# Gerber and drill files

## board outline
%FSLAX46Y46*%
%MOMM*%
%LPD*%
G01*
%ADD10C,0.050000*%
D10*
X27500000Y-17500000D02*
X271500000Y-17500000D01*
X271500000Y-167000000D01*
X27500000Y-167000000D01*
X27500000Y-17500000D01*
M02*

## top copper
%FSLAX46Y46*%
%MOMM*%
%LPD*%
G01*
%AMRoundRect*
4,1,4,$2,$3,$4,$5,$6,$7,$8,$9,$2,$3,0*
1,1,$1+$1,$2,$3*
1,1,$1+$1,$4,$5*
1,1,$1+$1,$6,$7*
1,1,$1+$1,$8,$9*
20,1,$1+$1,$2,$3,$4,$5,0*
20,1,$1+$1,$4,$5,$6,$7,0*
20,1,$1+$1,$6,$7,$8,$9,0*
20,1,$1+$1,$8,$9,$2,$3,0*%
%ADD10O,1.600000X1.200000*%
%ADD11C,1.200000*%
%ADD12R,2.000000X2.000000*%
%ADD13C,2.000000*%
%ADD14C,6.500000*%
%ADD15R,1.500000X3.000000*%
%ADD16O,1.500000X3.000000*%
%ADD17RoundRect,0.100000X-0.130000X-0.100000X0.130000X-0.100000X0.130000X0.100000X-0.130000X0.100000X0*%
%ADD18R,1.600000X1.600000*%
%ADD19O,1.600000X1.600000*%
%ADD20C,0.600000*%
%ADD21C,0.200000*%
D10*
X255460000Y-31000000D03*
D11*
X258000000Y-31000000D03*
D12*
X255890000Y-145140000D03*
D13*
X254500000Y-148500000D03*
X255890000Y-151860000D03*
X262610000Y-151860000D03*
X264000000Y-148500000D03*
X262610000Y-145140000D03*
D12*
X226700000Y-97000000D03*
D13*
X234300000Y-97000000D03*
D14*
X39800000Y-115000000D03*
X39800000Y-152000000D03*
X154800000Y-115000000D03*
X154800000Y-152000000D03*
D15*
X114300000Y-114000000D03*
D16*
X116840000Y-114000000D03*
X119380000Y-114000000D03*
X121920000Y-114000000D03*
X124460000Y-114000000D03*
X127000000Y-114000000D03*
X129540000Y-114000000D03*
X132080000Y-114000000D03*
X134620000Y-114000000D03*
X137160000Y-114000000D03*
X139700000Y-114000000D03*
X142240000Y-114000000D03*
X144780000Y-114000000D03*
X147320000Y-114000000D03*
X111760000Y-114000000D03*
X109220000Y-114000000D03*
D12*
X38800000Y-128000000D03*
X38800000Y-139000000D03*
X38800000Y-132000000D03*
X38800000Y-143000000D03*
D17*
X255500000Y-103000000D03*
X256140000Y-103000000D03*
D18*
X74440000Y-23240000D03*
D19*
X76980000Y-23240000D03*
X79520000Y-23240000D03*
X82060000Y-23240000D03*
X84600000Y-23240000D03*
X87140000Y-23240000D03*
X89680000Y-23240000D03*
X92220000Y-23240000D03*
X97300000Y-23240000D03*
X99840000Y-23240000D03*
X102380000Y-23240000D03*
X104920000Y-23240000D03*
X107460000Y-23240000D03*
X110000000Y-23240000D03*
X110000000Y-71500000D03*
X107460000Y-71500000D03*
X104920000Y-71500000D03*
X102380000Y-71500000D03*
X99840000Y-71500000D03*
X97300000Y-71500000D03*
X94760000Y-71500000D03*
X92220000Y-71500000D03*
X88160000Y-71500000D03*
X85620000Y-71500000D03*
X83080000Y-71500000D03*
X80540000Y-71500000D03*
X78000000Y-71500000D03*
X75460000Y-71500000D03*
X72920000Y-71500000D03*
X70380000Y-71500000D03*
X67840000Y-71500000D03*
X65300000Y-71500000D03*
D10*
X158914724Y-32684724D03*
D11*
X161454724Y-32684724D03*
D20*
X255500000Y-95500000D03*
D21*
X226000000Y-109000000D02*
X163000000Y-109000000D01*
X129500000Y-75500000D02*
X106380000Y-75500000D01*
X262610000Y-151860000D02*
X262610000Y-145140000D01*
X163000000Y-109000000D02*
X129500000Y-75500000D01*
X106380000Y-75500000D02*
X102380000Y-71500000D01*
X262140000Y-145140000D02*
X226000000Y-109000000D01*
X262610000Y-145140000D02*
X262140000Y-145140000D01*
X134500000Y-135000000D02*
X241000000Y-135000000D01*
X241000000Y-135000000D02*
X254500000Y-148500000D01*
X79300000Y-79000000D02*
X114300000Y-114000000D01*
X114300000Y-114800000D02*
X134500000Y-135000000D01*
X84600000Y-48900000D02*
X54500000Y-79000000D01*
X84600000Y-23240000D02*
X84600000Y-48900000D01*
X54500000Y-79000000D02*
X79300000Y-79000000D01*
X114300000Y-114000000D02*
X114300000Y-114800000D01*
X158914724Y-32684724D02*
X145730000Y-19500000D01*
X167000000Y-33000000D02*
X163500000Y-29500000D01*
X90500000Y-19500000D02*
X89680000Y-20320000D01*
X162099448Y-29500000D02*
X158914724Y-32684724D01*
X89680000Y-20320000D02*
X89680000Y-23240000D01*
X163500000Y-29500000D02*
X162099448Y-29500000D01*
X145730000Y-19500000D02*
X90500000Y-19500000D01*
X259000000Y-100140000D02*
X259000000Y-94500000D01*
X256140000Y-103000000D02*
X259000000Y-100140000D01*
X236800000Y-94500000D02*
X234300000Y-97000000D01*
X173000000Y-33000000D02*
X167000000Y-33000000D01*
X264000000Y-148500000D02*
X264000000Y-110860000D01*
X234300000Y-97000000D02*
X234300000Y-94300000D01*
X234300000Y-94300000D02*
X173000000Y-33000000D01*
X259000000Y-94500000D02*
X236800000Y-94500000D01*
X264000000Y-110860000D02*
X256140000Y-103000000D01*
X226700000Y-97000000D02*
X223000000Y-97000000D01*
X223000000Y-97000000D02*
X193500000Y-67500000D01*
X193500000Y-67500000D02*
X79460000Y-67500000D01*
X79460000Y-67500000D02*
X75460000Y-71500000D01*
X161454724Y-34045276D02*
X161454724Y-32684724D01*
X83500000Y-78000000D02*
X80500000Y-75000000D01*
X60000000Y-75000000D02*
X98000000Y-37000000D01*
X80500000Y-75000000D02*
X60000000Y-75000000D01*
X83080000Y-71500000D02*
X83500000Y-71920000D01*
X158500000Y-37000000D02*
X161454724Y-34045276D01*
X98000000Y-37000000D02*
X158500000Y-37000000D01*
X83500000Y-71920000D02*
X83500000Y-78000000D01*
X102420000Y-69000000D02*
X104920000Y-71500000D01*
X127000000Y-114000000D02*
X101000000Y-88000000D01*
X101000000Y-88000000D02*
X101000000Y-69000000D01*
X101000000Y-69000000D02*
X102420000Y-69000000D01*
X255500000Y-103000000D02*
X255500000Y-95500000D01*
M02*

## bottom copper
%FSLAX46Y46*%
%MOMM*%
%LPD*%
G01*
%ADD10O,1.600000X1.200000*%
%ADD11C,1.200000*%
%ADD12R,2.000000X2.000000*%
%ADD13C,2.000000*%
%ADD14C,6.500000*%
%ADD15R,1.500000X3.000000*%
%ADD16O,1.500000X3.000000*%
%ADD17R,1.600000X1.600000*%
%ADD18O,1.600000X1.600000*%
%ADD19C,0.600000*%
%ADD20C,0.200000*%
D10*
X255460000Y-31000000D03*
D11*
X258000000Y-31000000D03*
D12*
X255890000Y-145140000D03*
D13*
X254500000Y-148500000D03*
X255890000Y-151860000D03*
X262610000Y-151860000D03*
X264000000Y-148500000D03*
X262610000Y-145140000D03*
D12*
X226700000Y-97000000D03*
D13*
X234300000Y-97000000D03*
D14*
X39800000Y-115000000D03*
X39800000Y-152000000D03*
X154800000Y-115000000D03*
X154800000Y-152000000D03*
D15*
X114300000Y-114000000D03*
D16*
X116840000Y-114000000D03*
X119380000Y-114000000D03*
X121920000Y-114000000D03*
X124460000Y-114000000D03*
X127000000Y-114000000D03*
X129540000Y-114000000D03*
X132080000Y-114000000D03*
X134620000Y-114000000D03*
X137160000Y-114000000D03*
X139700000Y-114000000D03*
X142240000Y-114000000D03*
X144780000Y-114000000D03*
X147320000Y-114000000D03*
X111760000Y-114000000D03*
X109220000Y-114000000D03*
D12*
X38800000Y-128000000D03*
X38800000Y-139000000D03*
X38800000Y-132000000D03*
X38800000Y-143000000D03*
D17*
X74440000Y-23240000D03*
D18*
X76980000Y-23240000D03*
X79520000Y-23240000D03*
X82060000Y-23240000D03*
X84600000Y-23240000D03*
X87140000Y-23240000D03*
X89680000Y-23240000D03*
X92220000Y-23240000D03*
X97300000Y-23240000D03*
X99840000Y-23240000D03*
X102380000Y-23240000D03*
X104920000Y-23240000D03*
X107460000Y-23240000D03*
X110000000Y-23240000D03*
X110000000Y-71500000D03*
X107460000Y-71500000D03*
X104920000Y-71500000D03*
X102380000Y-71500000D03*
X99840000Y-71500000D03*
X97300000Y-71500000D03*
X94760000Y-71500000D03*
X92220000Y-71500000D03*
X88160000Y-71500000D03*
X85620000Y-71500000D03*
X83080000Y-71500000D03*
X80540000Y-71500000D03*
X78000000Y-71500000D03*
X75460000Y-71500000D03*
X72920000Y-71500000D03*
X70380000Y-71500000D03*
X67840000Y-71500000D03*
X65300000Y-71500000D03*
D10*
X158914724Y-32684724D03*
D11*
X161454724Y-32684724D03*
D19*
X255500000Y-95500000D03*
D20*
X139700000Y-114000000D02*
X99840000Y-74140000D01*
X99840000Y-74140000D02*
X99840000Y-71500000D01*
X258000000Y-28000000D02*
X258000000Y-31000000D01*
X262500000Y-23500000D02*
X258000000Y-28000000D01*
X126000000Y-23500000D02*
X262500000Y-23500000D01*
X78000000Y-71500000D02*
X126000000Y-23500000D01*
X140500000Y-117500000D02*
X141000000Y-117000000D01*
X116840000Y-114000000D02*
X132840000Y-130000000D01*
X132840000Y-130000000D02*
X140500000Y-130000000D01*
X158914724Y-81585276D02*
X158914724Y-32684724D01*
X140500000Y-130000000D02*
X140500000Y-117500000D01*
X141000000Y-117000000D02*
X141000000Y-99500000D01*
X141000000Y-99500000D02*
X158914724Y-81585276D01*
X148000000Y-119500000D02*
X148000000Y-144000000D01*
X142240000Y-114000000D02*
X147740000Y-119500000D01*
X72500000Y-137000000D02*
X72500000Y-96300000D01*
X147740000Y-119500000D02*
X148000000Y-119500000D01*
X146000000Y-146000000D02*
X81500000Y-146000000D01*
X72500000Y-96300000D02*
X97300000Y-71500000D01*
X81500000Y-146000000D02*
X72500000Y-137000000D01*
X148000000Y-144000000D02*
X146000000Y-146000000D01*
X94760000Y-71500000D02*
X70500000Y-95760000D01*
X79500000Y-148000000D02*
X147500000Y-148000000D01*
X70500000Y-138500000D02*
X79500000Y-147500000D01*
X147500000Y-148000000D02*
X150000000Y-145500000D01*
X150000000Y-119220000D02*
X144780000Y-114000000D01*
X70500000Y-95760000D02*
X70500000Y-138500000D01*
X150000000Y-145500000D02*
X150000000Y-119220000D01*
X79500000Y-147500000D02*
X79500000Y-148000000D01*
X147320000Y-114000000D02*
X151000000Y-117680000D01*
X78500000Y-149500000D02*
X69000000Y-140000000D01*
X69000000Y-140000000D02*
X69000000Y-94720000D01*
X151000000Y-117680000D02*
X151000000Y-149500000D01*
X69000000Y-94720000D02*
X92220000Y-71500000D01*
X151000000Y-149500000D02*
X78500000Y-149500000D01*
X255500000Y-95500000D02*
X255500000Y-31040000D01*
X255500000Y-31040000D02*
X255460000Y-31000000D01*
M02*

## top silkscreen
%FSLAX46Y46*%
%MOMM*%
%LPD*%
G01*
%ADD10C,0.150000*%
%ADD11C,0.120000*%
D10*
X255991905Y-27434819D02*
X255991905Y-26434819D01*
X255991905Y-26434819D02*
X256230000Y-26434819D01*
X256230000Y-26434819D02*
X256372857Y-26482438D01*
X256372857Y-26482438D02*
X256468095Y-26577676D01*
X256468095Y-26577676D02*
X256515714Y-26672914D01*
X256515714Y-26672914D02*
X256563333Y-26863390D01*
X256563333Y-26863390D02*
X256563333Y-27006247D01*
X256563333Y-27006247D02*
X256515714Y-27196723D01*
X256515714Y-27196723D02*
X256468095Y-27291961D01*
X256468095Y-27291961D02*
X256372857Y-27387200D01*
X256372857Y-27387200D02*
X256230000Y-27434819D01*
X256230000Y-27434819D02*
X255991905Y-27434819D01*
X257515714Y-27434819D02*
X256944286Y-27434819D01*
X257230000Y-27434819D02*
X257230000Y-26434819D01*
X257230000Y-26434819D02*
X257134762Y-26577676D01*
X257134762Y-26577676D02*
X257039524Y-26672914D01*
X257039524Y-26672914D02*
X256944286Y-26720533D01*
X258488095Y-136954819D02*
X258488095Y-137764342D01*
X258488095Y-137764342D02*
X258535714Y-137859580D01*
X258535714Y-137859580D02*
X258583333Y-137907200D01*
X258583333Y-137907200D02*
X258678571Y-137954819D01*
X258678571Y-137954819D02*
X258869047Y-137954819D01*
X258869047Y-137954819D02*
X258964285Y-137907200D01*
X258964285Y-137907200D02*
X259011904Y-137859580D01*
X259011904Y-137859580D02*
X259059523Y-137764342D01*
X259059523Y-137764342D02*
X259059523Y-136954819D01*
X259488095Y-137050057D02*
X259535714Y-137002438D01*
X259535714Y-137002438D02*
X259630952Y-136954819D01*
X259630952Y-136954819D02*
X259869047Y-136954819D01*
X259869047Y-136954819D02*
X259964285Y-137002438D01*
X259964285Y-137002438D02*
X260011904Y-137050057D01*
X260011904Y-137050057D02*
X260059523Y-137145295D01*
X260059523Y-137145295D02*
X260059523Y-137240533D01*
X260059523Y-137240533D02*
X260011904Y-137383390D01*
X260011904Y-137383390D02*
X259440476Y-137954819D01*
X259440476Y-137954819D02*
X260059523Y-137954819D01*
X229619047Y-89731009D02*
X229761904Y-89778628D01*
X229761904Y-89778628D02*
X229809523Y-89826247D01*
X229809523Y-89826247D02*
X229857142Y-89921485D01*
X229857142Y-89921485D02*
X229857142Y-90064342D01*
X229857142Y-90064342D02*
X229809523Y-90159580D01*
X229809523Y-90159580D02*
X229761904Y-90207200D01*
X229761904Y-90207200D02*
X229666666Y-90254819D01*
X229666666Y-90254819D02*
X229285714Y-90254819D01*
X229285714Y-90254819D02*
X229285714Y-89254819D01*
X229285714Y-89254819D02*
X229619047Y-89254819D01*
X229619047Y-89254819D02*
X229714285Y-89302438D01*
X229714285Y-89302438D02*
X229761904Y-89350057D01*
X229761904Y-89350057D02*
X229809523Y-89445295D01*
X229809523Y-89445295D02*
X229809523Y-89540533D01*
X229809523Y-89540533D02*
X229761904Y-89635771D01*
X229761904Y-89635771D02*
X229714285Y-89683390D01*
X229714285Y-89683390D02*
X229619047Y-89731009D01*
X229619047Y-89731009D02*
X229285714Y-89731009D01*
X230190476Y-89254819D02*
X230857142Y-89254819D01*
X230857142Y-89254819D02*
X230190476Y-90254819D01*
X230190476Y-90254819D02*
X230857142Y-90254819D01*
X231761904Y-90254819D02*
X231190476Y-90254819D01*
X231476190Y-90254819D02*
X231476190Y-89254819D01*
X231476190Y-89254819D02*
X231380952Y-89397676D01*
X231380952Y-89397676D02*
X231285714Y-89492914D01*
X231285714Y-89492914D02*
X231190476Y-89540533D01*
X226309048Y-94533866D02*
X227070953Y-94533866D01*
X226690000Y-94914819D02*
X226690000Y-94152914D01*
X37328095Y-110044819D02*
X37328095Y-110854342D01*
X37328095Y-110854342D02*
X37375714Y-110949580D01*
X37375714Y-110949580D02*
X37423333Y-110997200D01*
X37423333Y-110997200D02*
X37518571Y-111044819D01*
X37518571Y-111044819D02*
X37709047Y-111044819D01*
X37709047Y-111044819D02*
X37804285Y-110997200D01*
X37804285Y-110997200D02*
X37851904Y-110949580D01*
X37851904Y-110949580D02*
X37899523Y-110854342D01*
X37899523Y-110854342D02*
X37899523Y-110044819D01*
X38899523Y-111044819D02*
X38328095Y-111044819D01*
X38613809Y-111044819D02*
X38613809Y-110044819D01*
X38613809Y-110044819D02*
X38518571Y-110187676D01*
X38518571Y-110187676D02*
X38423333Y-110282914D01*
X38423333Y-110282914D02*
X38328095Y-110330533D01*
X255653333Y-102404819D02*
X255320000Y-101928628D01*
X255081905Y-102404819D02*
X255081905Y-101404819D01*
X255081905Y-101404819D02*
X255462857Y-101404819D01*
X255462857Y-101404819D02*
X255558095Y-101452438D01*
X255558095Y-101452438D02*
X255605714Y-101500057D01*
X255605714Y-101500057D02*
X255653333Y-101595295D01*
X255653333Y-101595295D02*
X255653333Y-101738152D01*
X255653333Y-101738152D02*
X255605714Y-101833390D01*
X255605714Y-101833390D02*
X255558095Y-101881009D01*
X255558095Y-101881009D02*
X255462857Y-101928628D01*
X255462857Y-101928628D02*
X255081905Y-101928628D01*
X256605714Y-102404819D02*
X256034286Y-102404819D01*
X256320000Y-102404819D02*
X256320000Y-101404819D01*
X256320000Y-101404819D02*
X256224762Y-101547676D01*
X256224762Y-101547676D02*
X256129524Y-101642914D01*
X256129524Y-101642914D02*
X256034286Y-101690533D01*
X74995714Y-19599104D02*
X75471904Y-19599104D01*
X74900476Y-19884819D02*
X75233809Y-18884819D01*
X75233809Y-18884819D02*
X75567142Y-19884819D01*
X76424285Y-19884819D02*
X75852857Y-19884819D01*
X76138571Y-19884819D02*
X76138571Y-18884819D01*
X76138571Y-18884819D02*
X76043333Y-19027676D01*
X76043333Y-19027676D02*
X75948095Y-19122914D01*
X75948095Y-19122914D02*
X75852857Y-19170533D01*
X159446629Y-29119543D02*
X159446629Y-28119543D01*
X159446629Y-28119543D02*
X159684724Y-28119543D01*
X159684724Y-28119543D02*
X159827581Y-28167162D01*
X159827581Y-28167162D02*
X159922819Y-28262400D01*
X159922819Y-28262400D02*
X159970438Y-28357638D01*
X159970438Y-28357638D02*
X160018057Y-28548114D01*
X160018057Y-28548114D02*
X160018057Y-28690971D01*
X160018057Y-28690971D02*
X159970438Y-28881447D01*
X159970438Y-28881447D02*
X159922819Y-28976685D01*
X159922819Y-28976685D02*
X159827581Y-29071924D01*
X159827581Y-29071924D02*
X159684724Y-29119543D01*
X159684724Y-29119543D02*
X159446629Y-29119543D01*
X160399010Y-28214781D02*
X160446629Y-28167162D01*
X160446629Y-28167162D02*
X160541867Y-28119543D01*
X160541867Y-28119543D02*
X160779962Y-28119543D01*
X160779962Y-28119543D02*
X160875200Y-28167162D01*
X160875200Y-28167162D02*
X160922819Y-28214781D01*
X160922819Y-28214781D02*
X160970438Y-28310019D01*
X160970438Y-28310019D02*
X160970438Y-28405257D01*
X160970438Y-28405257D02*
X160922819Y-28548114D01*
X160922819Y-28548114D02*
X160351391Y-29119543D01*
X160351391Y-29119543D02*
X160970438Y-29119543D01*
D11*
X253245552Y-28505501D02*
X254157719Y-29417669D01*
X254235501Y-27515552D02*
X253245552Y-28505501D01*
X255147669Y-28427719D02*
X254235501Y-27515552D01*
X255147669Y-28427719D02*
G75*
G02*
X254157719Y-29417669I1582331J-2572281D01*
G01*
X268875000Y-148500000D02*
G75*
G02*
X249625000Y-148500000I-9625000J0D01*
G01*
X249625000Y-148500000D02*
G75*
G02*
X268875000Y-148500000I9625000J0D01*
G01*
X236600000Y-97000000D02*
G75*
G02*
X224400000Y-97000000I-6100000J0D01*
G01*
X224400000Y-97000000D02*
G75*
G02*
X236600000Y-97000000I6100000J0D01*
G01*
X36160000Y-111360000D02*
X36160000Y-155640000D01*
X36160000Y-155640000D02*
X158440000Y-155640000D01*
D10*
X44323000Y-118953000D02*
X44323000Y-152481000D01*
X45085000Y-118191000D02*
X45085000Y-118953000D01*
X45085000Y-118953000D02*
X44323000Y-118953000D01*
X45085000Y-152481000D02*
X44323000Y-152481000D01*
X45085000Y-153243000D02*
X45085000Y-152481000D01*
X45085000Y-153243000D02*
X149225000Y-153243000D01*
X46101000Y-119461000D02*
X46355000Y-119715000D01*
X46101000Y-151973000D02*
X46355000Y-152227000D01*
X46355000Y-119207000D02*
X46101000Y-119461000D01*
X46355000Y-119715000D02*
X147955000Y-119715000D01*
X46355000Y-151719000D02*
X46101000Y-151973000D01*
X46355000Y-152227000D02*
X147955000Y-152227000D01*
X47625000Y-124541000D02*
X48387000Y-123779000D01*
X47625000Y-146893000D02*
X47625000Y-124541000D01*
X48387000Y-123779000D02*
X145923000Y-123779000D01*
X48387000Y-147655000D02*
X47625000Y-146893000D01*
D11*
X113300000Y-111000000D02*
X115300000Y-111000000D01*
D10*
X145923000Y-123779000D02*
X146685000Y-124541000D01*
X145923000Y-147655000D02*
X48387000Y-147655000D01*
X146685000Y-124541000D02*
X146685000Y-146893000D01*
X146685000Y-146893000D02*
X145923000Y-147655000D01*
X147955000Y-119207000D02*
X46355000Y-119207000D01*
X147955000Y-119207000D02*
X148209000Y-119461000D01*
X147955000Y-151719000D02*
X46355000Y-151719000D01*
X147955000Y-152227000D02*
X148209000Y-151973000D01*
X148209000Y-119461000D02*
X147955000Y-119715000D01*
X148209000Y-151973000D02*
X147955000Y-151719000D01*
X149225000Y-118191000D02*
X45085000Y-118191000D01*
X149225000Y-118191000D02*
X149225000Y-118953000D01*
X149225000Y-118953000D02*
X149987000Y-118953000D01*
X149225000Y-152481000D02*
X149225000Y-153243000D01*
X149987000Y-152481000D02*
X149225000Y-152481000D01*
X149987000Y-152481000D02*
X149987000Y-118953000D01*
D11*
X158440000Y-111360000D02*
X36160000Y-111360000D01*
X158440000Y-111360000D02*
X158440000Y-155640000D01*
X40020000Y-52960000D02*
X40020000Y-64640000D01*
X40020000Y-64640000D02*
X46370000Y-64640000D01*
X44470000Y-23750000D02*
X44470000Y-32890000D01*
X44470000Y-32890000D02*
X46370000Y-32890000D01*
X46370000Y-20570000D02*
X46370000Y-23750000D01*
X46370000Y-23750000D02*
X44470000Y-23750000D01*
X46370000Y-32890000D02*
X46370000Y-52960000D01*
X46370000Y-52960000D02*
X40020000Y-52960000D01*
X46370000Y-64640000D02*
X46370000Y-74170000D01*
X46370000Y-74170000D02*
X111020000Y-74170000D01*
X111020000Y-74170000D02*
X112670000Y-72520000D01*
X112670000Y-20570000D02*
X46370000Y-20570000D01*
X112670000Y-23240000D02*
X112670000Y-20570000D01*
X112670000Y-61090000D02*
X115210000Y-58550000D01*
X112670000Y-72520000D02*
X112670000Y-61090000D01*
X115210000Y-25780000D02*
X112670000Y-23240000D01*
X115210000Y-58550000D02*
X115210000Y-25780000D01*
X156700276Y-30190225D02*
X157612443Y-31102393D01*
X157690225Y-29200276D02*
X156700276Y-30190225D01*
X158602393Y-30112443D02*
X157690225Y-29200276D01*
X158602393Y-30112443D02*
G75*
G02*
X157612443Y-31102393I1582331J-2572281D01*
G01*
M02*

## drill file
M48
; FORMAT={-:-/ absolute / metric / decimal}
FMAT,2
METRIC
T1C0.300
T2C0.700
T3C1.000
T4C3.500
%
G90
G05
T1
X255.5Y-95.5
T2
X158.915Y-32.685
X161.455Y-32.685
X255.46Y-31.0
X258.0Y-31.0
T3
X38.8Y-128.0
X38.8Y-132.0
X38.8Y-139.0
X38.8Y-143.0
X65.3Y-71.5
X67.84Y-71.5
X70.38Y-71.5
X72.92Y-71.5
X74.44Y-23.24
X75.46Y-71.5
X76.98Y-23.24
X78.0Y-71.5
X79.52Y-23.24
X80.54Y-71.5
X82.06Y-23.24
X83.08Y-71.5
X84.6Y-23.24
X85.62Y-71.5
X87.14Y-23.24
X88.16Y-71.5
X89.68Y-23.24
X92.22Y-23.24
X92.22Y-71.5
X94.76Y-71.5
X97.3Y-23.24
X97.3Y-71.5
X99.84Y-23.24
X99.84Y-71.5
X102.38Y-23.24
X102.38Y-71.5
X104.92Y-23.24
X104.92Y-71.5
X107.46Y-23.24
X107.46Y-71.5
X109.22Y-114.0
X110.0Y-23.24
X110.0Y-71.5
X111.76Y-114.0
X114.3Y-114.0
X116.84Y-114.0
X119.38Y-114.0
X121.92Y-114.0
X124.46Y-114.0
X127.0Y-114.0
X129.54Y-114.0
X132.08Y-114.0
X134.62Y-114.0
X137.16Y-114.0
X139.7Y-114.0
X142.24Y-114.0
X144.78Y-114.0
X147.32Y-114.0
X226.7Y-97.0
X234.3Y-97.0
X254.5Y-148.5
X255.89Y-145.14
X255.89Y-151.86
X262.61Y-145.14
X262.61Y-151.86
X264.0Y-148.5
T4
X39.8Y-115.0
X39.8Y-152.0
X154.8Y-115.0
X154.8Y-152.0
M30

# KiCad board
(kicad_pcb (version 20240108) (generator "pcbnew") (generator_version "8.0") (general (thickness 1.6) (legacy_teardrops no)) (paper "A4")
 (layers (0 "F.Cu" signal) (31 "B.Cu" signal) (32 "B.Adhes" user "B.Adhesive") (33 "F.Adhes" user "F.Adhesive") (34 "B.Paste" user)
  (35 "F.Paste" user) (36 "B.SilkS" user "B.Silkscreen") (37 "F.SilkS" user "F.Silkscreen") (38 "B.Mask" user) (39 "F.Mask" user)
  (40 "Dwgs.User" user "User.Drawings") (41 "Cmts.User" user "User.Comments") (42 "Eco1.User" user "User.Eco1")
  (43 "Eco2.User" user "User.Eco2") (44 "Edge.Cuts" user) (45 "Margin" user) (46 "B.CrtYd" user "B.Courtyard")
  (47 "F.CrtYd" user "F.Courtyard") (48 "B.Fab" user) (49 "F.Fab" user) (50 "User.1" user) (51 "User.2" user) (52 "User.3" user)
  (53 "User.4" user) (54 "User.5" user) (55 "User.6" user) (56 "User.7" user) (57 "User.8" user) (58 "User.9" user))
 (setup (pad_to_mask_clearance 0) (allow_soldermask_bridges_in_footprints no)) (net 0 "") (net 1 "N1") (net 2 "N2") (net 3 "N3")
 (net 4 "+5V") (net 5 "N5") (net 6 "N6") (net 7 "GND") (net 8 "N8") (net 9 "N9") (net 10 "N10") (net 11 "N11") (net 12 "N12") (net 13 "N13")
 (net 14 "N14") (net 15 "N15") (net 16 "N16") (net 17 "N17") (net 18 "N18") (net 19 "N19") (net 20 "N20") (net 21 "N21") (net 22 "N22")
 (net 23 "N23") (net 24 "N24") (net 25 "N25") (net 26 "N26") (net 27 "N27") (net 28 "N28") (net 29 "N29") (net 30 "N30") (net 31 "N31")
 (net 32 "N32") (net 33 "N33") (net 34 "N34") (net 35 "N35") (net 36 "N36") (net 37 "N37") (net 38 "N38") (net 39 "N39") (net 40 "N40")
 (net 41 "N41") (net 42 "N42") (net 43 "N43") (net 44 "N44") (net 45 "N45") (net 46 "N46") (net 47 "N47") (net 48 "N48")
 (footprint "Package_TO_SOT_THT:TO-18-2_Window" (layer "F.Cu") (at 255.46 31)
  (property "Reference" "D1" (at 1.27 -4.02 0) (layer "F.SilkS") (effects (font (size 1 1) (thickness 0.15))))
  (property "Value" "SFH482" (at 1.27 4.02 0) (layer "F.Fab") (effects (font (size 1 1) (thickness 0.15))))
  (fp_line (start -2.214448 -2.494499) (end -1.302281 -1.582331) (stroke (width 0.12) (type solid)) (layer "F.SilkS"))
  (fp_line (start -1.224499 -3.484448) (end -2.214448 -2.494499) (stroke (width 0.12) (type solid)) (layer "F.SilkS"))
  (fp_line (start -0.312331 -2.572281) (end -1.224499 -3.484448) (stroke (width 0.12) (type solid)) (layer "F.SilkS"))
  (fp_arc (start -0.312331 -2.572281) (mid 3.405463 2.135463) (end -1.302281 -1.582331) (stroke (width 0.12) (type solid)) (layer "F.SilkS"))
  (pad "1" thru_hole oval (at 0 0) (size 1.6 1.2) (drill 0.7) (layers "*.Cu" "*.Mask") (remove_unused_layers no) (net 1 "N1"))
  (pad "2" thru_hole circle (at 2.54 0) (size 1.2 1.2) (drill 0.7) (layers "*.Cu" "*.Mask") (remove_unused_layers no) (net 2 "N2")))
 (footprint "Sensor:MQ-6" (layer "F.Cu") (at 255.89 145.14)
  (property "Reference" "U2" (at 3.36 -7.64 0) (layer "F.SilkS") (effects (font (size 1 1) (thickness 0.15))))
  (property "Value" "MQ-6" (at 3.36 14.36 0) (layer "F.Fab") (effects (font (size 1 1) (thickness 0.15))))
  (fp_circle (center 3.36 3.36) (end 12.985 3.36) (stroke (width 0.12) (type solid)) (fill none) (layer "F.SilkS"))
  (pad "1" thru_hole rect (at 0 0) (size 2 2) (drill 1) (layers "*.Cu" "*.Mask") (remove_unused_layers no) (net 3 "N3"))
  (pad "2" thru_hole circle (at -1.39 3.36) (size 2 2) (drill 1) (layers "*.Cu" "*.Mask") (remove_unused_layers no) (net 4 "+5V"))
  (pad "3" thru_hole circle (at 0 6.72 90) (size 2 2) (drill 1) (layers "*.Cu" "*.Mask") (remove_unused_layers no) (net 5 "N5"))
  (pad "4" thru_hole circle (at 6.72 6.72 180) (size 2 2) (drill 1) (layers "*.Cu" "*.Mask") (remove_unused_layers no) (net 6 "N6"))
  (pad "5" thru_hole circle (at 8.11 3.36) (size 2 2) (drill 1) (layers "*.Cu" "*.Mask") (remove_unused_layers no) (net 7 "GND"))
  (pad "6" thru_hole circle (at 6.72 0 270) (size 2 2) (drill 1) (layers "*.Cu" "*.Mask") (remove_unused_layers no) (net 6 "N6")))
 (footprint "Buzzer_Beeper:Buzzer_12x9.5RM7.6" (layer "F.Cu") (at 226.7 97)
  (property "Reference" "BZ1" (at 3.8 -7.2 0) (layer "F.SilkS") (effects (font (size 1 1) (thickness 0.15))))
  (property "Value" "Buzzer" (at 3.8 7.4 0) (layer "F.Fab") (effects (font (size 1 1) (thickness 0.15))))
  (fp_circle (center 3.8 0) (end 9.9 0) (stroke (width 0.12) (type solid)) (fill none) (layer "F.SilkS"))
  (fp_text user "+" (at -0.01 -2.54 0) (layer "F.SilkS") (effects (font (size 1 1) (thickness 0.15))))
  (pad "1" thru_hole rect (at 0 0) (size 2 2) (drill 1) (layers "*.Cu" "*.Mask") (remove_unused_layers no) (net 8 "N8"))
  (pad "2" thru_hole circle (at 7.6 0) (size 2 2) (drill 1) (layers "*.Cu" "*.Mask") (remove_unused_layers no) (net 7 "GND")))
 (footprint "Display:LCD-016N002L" (layer "F.Cu") (at 114.3 114)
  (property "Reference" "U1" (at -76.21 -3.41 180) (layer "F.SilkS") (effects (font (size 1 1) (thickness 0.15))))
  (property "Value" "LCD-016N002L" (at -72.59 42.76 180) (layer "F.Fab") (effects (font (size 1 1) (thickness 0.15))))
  (fp_line (start -78.14 -2.64) (end -78.14 41.64) (stroke (width 0.12) (type solid)) (layer "F.SilkS"))
  (fp_line (start -78.14 41.64) (end 44.14 41.64) (stroke (width 0.12) (type solid)) (layer "F.SilkS"))
  (fp_line (start -69.977 4.953) (end -69.977 38.481) (stroke (width 0.15) (type solid)) (layer "F.SilkS"))
  (fp_line (start -69.215 4.191) (end -69.215 4.953) (stroke (width 0.15) (type solid)) (layer "F.SilkS"))
  (fp_line (start -69.215 4.953) (end -69.977 4.953) (stroke (width 0.15) (type solid)) (layer "F.SilkS"))
  (fp_line (start -69.215 38.481) (end -69.977 38.481) (stroke (width 0.15) (type solid)) (layer "F.SilkS"))
  (fp_line (start -69.215 39.243) (end -69.215 38.481) (stroke (width 0.15) (type solid)) (layer "F.SilkS"))
  (fp_line (start -69.215 39.243) (end 34.925 39.243) (stroke (width 0.15) (type solid)) (layer "F.SilkS"))
  (fp_line (start -68.199 5.461) (end -67.945 5.715) (stroke (width 0.15) (type solid)) (layer "F.SilkS"))
  (fp_line (start -68.199 37.973) (end -67.945 38.227) (stroke (width 0.15) (type solid)) (layer "F.SilkS"))
  (fp_line (start -67.945 5.207) (end -68.199 5.461) (stroke (width 0.15) (type solid)) (layer "F.SilkS"))
  (fp_line (start -67.945 5.715) (end 33.655 5.715) (stroke (width 0.15) (type solid)) (layer "F.SilkS"))
  (fp_line (start -67.945 37.719) (end -68.199 37.973) (stroke (width 0.15) (type solid)) (layer "F.SilkS"))
  (fp_line (start -67.945 38.227) (end 33.655 38.227) (stroke (width 0.15) (type solid)) (layer "F.SilkS"))
  (fp_line (start -66.675 10.541) (end -65.913 9.779) (stroke (width 0.15) (type solid)) (layer "F.SilkS"))
  (fp_line (start -66.675 32.893) (end -66.675 10.541) (stroke (width 0.15) (type solid)) (layer "F.SilkS"))
  (fp_line (start -65.913 9.779) (end 31.623 9.779) (stroke (width 0.15) (type solid)) (layer "F.SilkS"))
  (fp_line (start -65.913 33.655) (end -66.675 32.893) (stroke (width 0.15) (type solid)) (layer "F.SilkS"))
  (fp_line (start -1 -3) (end 1 -3) (stroke (width 0.12) (type solid)) (layer "F.SilkS"))
  (fp_line (start 31.623 9.779) (end 32.385 10.541) (stroke (width 0.15) (type solid)) (layer "F.SilkS"))
  (fp_line (start 31.623 33.655) (end -65.913 33.655) (stroke (width 0.15) (type solid)) (layer "F.SilkS"))
  (fp_line (start 32.385 10.541) (end 32.385 32.893) (stroke (width 0.15) (type solid)) (layer "F.SilkS"))
  (fp_line (start 32.385 32.893) (end 31.623 33.655) (stroke (width 0.15) (type solid)) (layer "F.SilkS"))
  (fp_line (start 33.655 5.207) (end -67.945 5.207) (stroke (width 0.15) (type solid)) (layer "F.SilkS"))
  (fp_line (start 33.655 5.207) (end 33.909 5.461) (stroke (width 0.15) (type solid)) (layer "F.SilkS"))
  (fp_line (start 33.655 37.719) (end -67.945 37.719) (stroke (width 0.15) (type solid)) (layer "F.SilkS"))
  (fp_line (start 33.655 38.227) (end 33.909 37.973) (stroke (width 0.15) (type solid)) (layer "F.SilkS"))
  (fp_line (start 33.909 5.461) (end 33.655 5.715) (stroke (width 0.15) (type solid)) (layer "F.SilkS"))
  (fp_line (start 33.909 37.973) (end 33.655 37.719) (stroke (width 0.15) (type solid)) (layer "F.SilkS"))
  (fp_line (start 34.925 4.191) (end -69.215 4.191) (stroke (width 0.15) (type solid)) (layer "F.SilkS"))
  (fp_line (start 34.925 4.191) (end 34.925 4.953) (stroke (width 0.15) (type solid)) (layer "F.SilkS"))
  (fp_line (start 34.925 4.953) (end 35.687 4.953) (stroke (width 0.15) (type solid)) (layer "F.SilkS"))
  (fp_line (start 34.925 38.481) (end 34.925 39.243) (stroke (width 0.15) (type solid)) (layer "F.SilkS"))
  (fp_line (start 35.687 38.481) (end 34.925 38.481) (stroke (width 0.15) (type solid)) (layer "F.SilkS"))
  (fp_line (start 35.687 38.481) (end 35.687 4.953) (stroke (width 0.15) (type solid)) (layer "F.SilkS"))
  (fp_line (start 44.14 -2.64) (end -78.14 -2.64) (stroke (width 0.12) (type solid)) (layer "F.SilkS"))
  (fp_line (start 44.14 -2.64) (end 44.14 41.64) (stroke (width 0.12) (type solid)) (layer "F.SilkS"))
  (pad "" thru_hole circle (at -74.5 1 180) (size 6.5 6.5) (drill 3.5) (layers "*.Cu" "*.Mask") (remove_unused_layers no))
  (pad "" thru_hole circle (at -74.5 38 180) (size 6.5 6.5) (drill 3.5) (layers "*.Cu" "*.Mask") (remove_unused_layers no))
  (pad "" thru_hole circle (at 40.5 1 180) (size 6.5 6.5) (drill 3.5) (layers "*.Cu" "*.Mask") (remove_unused_layers no))
  (pad "" thru_hole circle (at 40.5 38 180) (size 6.5 6.5) (drill 3.5) (layers "*.Cu" "*.Mask") (remove_unused_layers no))
  (pad "1" thru_hole rect (at 0 0 180) (size 1.5 3) (drill 1) (layers "*.Cu" "*.Mask") (remove_unused_layers no) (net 4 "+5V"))
  (pad "2" thru_hole oval (at 2.54 0 180) (size 1.5 3) (drill 1) (layers "*.Cu" "*.Mask") (remove_unused_layers no) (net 7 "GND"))
  (pad "3" thru_hole oval (at 5.08 0 180) (size 1.5 3) (drill 1) (layers "*.Cu" "*.Mask") (remove_unused_layers no) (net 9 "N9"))
  (pad "4" thru_hole oval (at 7.62 0 180) (size 1.5 3) (drill 1) (layers "*.Cu" "*.Mask") (remove_unused_layers no) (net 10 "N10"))
  (pad "5" thru_hole oval (at 10.16 0 180) (size 1.5 3) (drill 1) (layers "*.Cu" "*.Mask") (remove_unused_layers no) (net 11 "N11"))
  (pad "6" thru_hole oval (at 12.7 0 180) (size 1.5 3) (drill 1) (layers "*.Cu" "*.Mask") (remove_unused_layers no) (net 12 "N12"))
  (pad "7" thru_hole oval (at 15.24 0 180) (size 1.5 3) (drill 1) (layers "*.Cu" "*.Mask") (remove_unused_layers no) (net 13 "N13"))
  (pad "8" thru_hole oval (at 17.78 0 180) (size 1.5 3) (drill 1) (layers "*.Cu" "*.Mask") (remove_unused_layers no) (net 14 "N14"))
  (pad "9" thru_hole oval (at 20.32 0 180) (size 1.5 3) (drill 1) (layers "*.Cu" "*.Mask") (remove_unused_layers no) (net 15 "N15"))
  (pad "10" thru_hole oval (at 22.86 0 180) (size 1.5 3) (drill 1) (layers "*.Cu" "*.Mask") (remove_unused_layers no) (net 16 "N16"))
  (pad "11" thru_hole oval (at 25.4 0 180) (size 1.5 3) (drill 1) (layers "*.Cu" "*.Mask") (remove_unused_layers no) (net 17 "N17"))
  (pad "12" thru_hole oval (at 27.94 0 180) (size 1.5 3) (drill 1) (layers "*.Cu" "*.Mask") (remove_unused_layers no) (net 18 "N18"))
  (pad "13" thru_hole oval (at 30.48 0 180) (size 1.5 3) (drill 1) (layers "*.Cu" "*.Mask") (remove_unused_layers no) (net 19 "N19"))
  (pad "14" thru_hole oval (at 33.02 0 180) (size 1.5 3) (drill 1) (layers "*.Cu" "*.Mask") (remove_unused_layers no) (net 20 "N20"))
  (pad "15" thru_hole oval (at -2.54 0 180) (size 1.5 3) (drill 1) (layers "*.Cu" "*.Mask") (remove_unused_layers no) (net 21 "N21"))
  (pad "16" thru_hole oval (at -5.08 0 180) (size 1.5 3) (drill 1) (layers "*.Cu" "*.Mask") (remove_unused_layers no) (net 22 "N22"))
  (pad "A1" thru_hole rect (at -75.5 14 180) (size 2 2) (drill 1) (layers "*.Cu" "*.Mask") (remove_unused_layers no) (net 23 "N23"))
  (pad "A2" thru_hole rect (at -75.5 25 180) (size 2 2) (drill 1) (layers "*.Cu" "*.Mask") (remove_unused_layers no) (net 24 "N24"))
  (pad "K1" thru_hole rect (at -75.5 18 180) (size 2 2) (drill 1) (layers "*.Cu" "*.Mask") (remove_unused_layers no) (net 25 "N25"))
  (pad "K2" thru_hole rect (at -75.5 29 180) (size 2 2) (drill 1) (layers "*.Cu" "*.Mask") (remove_unused_layers no) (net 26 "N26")))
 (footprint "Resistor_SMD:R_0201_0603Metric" (layer "F.Cu") (at 255.82 103)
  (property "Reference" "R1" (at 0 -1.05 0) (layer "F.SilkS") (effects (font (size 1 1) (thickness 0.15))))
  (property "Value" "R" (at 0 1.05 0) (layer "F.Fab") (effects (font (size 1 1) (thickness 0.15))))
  (pad "" smd roundrect (at -0.345 0) (size 0.318 0.36) (layers "F.Paste") (roundrect_rratio 0.25))
  (pad "" smd roundrect (at 0.345 0) (size 0.318 0.36) (layers "F.Paste") (roundrect_rratio 0.25))
  (pad "1" smd roundrect (at -0.32 0) (size 0.46 0.4) (layers "F.Cu" "F.Mask") (roundrect_rratio 0.25) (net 1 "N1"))
  (pad "2" smd roundrect (at 0.32 0) (size 0.46 0.4) (layers "F.Cu" "F.Mask") (roundrect_rratio 0.25) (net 7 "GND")))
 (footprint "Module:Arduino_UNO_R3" (layer "F.Cu") (at 74.44 23.24)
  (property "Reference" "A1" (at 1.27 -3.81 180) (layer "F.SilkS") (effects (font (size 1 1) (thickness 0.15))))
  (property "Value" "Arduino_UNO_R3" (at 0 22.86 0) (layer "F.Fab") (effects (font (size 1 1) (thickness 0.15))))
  (fp_line (start -34.42 29.72) (end -34.42 41.4) (stroke (width 0.12) (type solid)) (layer "F.SilkS"))
  (fp_line (start -34.42 41.4) (end -28.07 41.4) (stroke (width 0.12) (type solid)) (layer "F.SilkS"))
  (fp_line (start -29.97 0.51) (end -29.97 9.65) (stroke (width 0.12) (type solid)) (layer "F.SilkS"))
  (fp_line (start -29.97 9.65) (end -28.07 9.65) (stroke (width 0.12) (type solid)) (layer "F.SilkS"))
  (fp_line (start -28.07 -2.67) (end -28.07 0.51) (stroke (width 0.12) (type solid)) (layer "F.SilkS"))
  (fp_line (start -28.07 0.51) (end -29.97 0.51) (stroke (width 0.12) (type solid)) (layer "F.SilkS"))
  (fp_line (start -28.07 9.65) (end -28.07 29.72) (stroke (width 0.12) (type solid)) (layer "F.SilkS"))
  (fp_line (start -28.07 29.72) (end -34.42 29.72) (stroke (width 0.12) (type solid)) (layer "F.SilkS"))
  (fp_line (start -28.07 41.4) (end -28.07 50.93) (stroke (width 0.12) (type solid)) (layer "F.SilkS"))
  (fp_line (start -28.07 50.93) (end 36.58 50.93) (stroke (width 0.12) (type solid)) (layer "F.SilkS"))
  (fp_line (start 36.58 50.93) (end 38.23 49.28) (stroke (width 0.12) (type solid)) (layer "F.SilkS"))
  (fp_line (start 38.23 -2.67) (end -28.07 -2.67) (stroke (width 0.12) (type solid)) (layer "F.SilkS"))
  (fp_line (start 38.23 0) (end 38.23 -2.67) (stroke (width 0.12) (type solid)) (layer "F.SilkS"))
  (fp_line (start 38.23 37.85) (end 40.77 35.31) (stroke (width 0.12) (type solid)) (layer "F.SilkS"))
  (fp_line (start 38.23 49.28) (end 38.23 37.85) (stroke (width 0.12) (type solid)) (layer "F.SilkS"))
  (fp_line (start 40.77 2.54) (end 38.23 0) (stroke (width 0.12) (type solid)) (layer "F.SilkS"))
  (fp_line (start 40.77 35.31) (end 40.77 2.54) (stroke (width 0.12) (type solid)) (layer "F.SilkS"))
  (pad "1" thru_hole rect (at 0 0 90) (size 1.6 1.6) (drill 1) (layers "*.Cu" "*.Mask") (remove_unused_layers no) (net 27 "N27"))
  (pad "2" thru_hole oval (at 2.54 0 90) (size 1.6 1.6) (drill 1) (layers "*.Cu" "*.Mask") (remove_unused_layers no) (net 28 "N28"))
  (pad "3" thru_hole oval (at 5.08 0 90) (size 1.6 1.6) (drill 1) (layers "*.Cu" "*.Mask") (remove_unused_layers no) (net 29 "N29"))
  (pad "4" thru_hole oval (at 7.62 0 90) (size 1.6 1.6) (drill 1) (layers "*.Cu" "*.Mask") (remove_unused_layers no) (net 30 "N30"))
  (pad "5" thru_hole oval (at 10.16 0 90) (size 1.6 1.6) (drill 1) (layers "*.Cu" "*.Mask") (remove_unused_layers no) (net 4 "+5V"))
  (pad "6" thru_hole oval (at 12.7 0 90) (size 1.6 1.6) (drill 1) (layers "*.Cu" "*.Mask") (remove_unused_layers no) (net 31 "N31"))
  (pad "7" thru_hole oval (at 15.24 0 90) (size 1.6 1.6) (drill 1) (layers "*.Cu" "*.Mask") (remove_unused_layers no) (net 7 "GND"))
  (pad "8" thru_hole oval (at 17.78 0 90) (size 1.6 1.6) (drill 1) (layers "*.Cu" "*.Mask") (remove_unused_layers no) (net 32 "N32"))
  (pad "9" thru_hole oval (at 22.86 0 90) (size 1.6 1.6) (drill 1) (layers "*.Cu" "*.Mask") (remove_unused_layers no) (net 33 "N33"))
  (pad "10" thru_hole oval (at 25.4 0 90) (size 1.6 1.6) (drill 1) (layers "*.Cu" "*.Mask") (remove_unused_layers no) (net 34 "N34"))
  (pad "11" thru_hole oval (at 27.94 0 90) (size 1.6 1.6) (drill 1) (layers "*.Cu" "*.Mask") (remove_unused_layers no) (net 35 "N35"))
  (pad "12" thru_hole oval (at 30.48 0 90) (size 1.6 1.6) (drill 1) (layers "*.Cu" "*.Mask") (remove_unused_layers no) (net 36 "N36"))
  (pad "13" thru_hole oval (at 33.02 0 90) (size 1.6 1.6) (drill 1) (layers "*.Cu" "*.Mask") (remove_unused_layers no) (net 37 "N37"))
  (pad "14" thru_hole oval (at 35.56 0 90) (size 1.6 1.6) (drill 1) (layers "*.Cu" "*.Mask") (remove_unused_layers no) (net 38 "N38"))
  (pad "15" thru_hole oval (at 35.56 48.26 90) (size 1.6 1.6) (drill 1) (layers "*.Cu" "*.Mask") (remove_unused_layers no) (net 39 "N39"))
  (pad "16" thru_hole oval (at 33.02 48.26 90) (size 1.6 1.6) (drill 1) (layers "*.Cu" "*.Mask") (remove_unused_layers no) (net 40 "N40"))
  (pad "17" thru_hole oval (at 30.48 48.26 90) (size 1.6 1.6) (drill 1) (layers "*.Cu" "*.Mask") (remove_unused_layers no) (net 12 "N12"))
  (pad "18" thru_hole oval (at 27.94 48.26 90) (size 1.6 1.6) (drill 1) (layers "*.Cu" "*.Mask") (remove_unused_layers no) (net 6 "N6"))
  (pad "19" thru_hole oval (at 25.4 48.26 90) (size 1.6 1.6) (drill 1) (layers "*.Cu" "*.Mask") (remove_unused_layers no) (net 17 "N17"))
  (pad "20" thru_hole oval (at 22.86 48.26 90) (size 1.6 1.6) (drill 1) (layers "*.Cu" "*.Mask") (remove_unused_layers no) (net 18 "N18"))
  (pad "21" thru_hole oval (at 20.32 48.26 90) (size 1.6 1.6) (drill 1) (layers "*.Cu" "*.Mask") (remove_unused_layers no) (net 19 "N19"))
  (pad "22" thru_hole oval (at 17.78 48.26 90) (size 1.6 1.6) (drill 1) (layers "*.Cu" "*.Mask") (remove_unused_layers no) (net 20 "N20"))
  (pad "23" thru_hole oval (at 13.72 48.26 90) (size 1.6 1.6) (drill 1) (layers "*.Cu" "*.Mask") (remove_unused_layers no) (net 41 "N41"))
  (pad "24" thru_hole oval (at 11.18 48.26 90) (size 1.6 1.6) (drill 1) (layers "*.Cu" "*.Mask") (remove_unused_layers no) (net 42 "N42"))
  (pad "25" thru_hole oval (at 8.64 48.26 90) (size 1.6 1.6) (drill 1) (layers "*.Cu" "*.Mask") (remove_unused_layers no) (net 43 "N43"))
  (pad "26" thru_hole oval (at 6.1 48.26 90) (size 1.6 1.6) (drill 1) (layers "*.Cu" "*.Mask") (remove_unused_layers no) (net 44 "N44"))
  (pad "27" thru_hole oval (at 3.56 48.26 90) (size 1.6 1.6) (drill 1) (layers "*.Cu" "*.Mask") (remove_unused_layers no) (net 2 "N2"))
  (pad "28" thru_hole oval (at 1.02 48.26 90) (size 1.6 1.6) (drill 1) (layers "*.Cu" "*.Mask") (remove_unused_layers no) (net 8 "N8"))
  (pad "29" thru_hole oval (at -1.52 48.26 90) (size 1.6 1.6) (drill 1) (layers "*.Cu" "*.Mask") (remove_unused_layers no) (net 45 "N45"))
  (pad "30" thru_hole oval (at -4.06 48.26 90) (size 1.6 1.6) (drill 1) (layers "*.Cu" "*.Mask") (remove_unused_layers no) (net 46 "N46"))
  (pad "31" thru_hole oval (at -6.6 48.26 90) (size 1.6 1.6) (drill 1) (layers "*.Cu" "*.Mask") (remove_unused_layers no) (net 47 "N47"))
  (pad "32" thru_hole oval (at -9.14 48.26 90) (size 1.6 1.6) (drill 1) (layers "*.Cu" "*.Mask") (remove_unused_layers no) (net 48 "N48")))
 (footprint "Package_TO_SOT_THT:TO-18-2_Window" (layer "F.Cu") (at 158.914724 32.684724)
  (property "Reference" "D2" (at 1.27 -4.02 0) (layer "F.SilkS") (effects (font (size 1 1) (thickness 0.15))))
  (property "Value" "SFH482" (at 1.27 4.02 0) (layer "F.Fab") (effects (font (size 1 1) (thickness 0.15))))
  (fp_line (start -2.214448 -2.494499) (end -1.302281 -1.582331) (stroke (width 0.12) (type solid)) (layer "F.SilkS"))
  (fp_line (start -1.224499 -3.484448) (end -2.214448 -2.494499) (stroke (width 0.12) (type solid)) (layer "F.SilkS"))
  (fp_line (start -0.312331 -2.572281) (end -1.224499 -3.484448) (stroke (width 0.12) (type solid)) (layer "F.SilkS"))
  (fp_arc (start -0.312331 -2.572281) (mid 3.405463 2.135463) (end -1.302281 -1.582331) (stroke (width 0.12) (type solid)) (layer "F.SilkS"))
  (pad "1" thru_hole oval (at 0 0) (size 1.6 1.2) (drill 0.7) (layers "*.Cu" "*.Mask") (remove_unused_layers no) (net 7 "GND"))
  (pad "2" thru_hole circle (at 2.54 0) (size 1.2 1.2) (drill 0.7) (layers "*.Cu" "*.Mask") (remove_unused_layers no) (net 43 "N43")))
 (gr_rect (start 27.5 17.5) (end 271.5 167) (stroke (width 0.05) (type default)) (fill none) (layer "Edge.Cuts"))
 (segment (start 139.7 114) (end 99.84 74.14) (width 0.2) (layer "B.Cu") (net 17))
 (segment (start 99.84 74.14) (end 99.84 71.5) (width 0.2) (layer "B.Cu") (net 17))
 (segment (start 226 109) (end 163 109) (width 0.2) (layer "F.Cu") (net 6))
 (segment (start 129.5 75.5) (end 106.38 75.5) (width 0.2) (layer "F.Cu") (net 6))
 (segment (start 262.61 151.86) (end 262.61 145.14) (width 0.2) (layer "F.Cu") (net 6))
 (segment (start 163 109) (end 129.5 75.5) (width 0.2) (layer "F.Cu") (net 6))
 (segment (start 106.38 75.5) (end 102.38 71.5) (width 0.2) (layer "F.Cu") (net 6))
 (segment (start 262.14 145.14) (end 226 109) (width 0.2) (layer "F.Cu") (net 6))
 (segment (start 262.61 145.14) (end 262.14 145.14) (width 0.2) (layer "F.Cu") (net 6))
 (segment (start 134.5 135) (end 241 135) (width 0.2) (layer "F.Cu") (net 4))
 (segment (start 241 135) (end 254.5 148.5) (width 0.2) (layer "F.Cu") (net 4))
 (segment (start 79.3 79) (end 114.3 114) (width 0.2) (layer "F.Cu") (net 4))
 (segment (start 114.3 114.8) (end 134.5 135) (width 0.2) (layer "F.Cu") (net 4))
 (segment (start 84.6 48.9) (end 54.5 79) (width 0.2) (layer "F.Cu") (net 4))
 (segment (start 84.6 23.24) (end 84.6 48.9) (width 0.2) (layer "F.Cu") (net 4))
 (segment (start 54.5 79) (end 79.3 79) (width 0.2) (layer "F.Cu") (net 4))
 (segment (start 114.3 114) (end 114.3 114.8) (width 0.2) (layer "F.Cu") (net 4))
 (segment (start 258 28) (end 258 31) (width 0.2) (layer "B.Cu") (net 2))
 (segment (start 262.5 23.5) (end 258 28) (width 0.2) (layer "B.Cu") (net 2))
 (segment (start 126 23.5) (end 262.5 23.5) (width 0.2) (layer "B.Cu") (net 2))
 (segment (start 78 71.5) (end 126 23.5) (width 0.2) (layer "B.Cu") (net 2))
 (segment (start 158.914724 32.684724) (end 145.73 19.5) (width 0.2) (layer "F.Cu") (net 7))
 (segment (start 167 33) (end 163.5 29.5) (width 0.2) (layer "F.Cu") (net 7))
 (segment (start 90.5 19.5) (end 89.68 20.32) (width 0.2) (layer "F.Cu") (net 7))
 (segment (start 162.099448 29.5) (end 158.914724 32.684724) (width 0.2) (layer "F.Cu") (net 7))
 (segment (start 89.68 20.32) (end 89.68 23.24) (width 0.2) (layer "F.Cu") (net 7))
 (segment (start 163.5 29.5) (end 162.099448 29.5) (width 0.2) (layer "F.Cu") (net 7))
 (segment (start 145.73 19.5) (end 90.5 19.5) (width 0.2) (layer "F.Cu") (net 7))
 (segment (start 259 100.14) (end 259 94.5) (width 0.2) (layer "F.Cu") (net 7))
 (segment (start 256.14 103) (end 259 100.14) (width 0.2) (layer "F.Cu") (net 7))
 (segment (start 236.8 94.5) (end 234.3 97) (width 0.2) (layer "F.Cu") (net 7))
 (segment (start 173 33) (end 167 33) (width 0.2) (layer "F.Cu") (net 7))
 (segment (start 264 148.5) (end 264 110.86) (width 0.2) (layer "F.Cu") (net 7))
 (segment (start 234.3 97) (end 234.3 94.3) (width 0.2) (layer "F.Cu") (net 7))
 (segment (start 234.3 94.3) (end 173 33) (width 0.2) (layer "F.Cu") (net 7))
 (segment (start 259 94.5) (end 236.8 94.5) (width 0.2) (layer "F.Cu") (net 7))
 (segment (start 264 110.86) (end 256.14 103) (width 0.2) (layer "F.Cu") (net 7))
 (segment (start 140.5 117.5) (end 141 117) (width 0.2) (layer "B.Cu") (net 7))
 (segment (start 116.84 114) (end 132.84 130) (width 0.2) (layer "B.Cu") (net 7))
 (segment (start 132.84 130) (end 140.5 130) (width 0.2) (layer "B.Cu") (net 7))
 (segment (start 158.914724 81.585276) (end 158.914724 32.684724) (width 0.2) (layer "B.Cu") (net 7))
 (segment (start 140.5 130) (end 140.5 117.5) (width 0.2) (layer "B.Cu") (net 7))
 (segment (start 141 117) (end 141 99.5) (width 0.2) (layer "B.Cu") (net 7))
 (segment (start 141 99.5) (end 158.914724 81.585276) (width 0.2) (layer "B.Cu") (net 7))
 (segment (start 148 119.5) (end 148 144) (width 0.2) (layer "B.Cu") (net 18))
 (segment (start 142.24 114) (end 147.74 119.5) (width 0.2) (layer "B.Cu") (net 18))
 (segment (start 72.5 137) (end 72.5 96.3) (width 0.2) (layer "B.Cu") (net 18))
 (segment (start 147.74 119.5) (end 148 119.5) (width 0.2) (layer "B.Cu") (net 18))
 (segment (start 146 146) (end 81.5 146) (width 0.2) (layer "B.Cu") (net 18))
 (segment (start 72.5 96.3) (end 97.3 71.5) (width 0.2) (layer "B.Cu") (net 18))
 (segment (start 81.5 146) (end 72.5 137) (width 0.2) (layer "B.Cu") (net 18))
 (segment (start 148 144) (end 146 146) (width 0.2) (layer "B.Cu") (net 18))
 (segment (start 226.7 97) (end 223 97) (width 0.2) (layer "F.Cu") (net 8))
 (segment (start 223 97) (end 193.5 67.5) (width 0.2) (layer "F.Cu") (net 8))
 (segment (start 193.5 67.5) (end 79.46 67.5) (width 0.2) (layer "F.Cu") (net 8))
 (segment (start 79.46 67.5) (end 75.46 71.5) (width 0.2) (layer "F.Cu") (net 8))
 (segment (start 161.454724 34.045276) (end 161.454724 32.684724) (width 0.2) (layer "F.Cu") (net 43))
 (segment (start 83.5 78) (end 80.5 75) (width 0.2) (layer "F.Cu") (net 43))
 (segment (start 60 75) (end 98 37) (width 0.2) (layer "F.Cu") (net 43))
 (segment (start 80.5 75) (end 60 75) (width 0.2) (layer "F.Cu") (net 43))
 (segment (start 83.08 71.5) (end 83.5 71.92) (width 0.2) (layer "F.Cu") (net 43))
 (segment (start 158.5 37) (end 161.454724 34.045276) (width 0.2) (layer "F.Cu") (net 43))
 (segment (start 98 37) (end 158.5 37) (width 0.2) (layer "F.Cu") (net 43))
 (segment (start 83.5 71.92) (end 83.5 78) (width 0.2) (layer "F.Cu") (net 43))
 (segment (start 94.76 71.5) (end 70.5 95.76) (width 0.2) (layer "B.Cu") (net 19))
 (segment (start 79.5 148) (end 147.5 148) (width 0.2) (layer "B.Cu") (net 19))
 (segment (start 70.5 138.5) (end 79.5 147.5) (width 0.2) (layer "B.Cu") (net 19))
 (segment (start 147.5 148) (end 150 145.5) (width 0.2) (layer "B.Cu") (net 19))
 (segment (start 150 119.22) (end 144.78 114) (width 0.2) (layer "B.Cu") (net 19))
 (segment (start 70.5 95.76) (end 70.5 138.5) (width 0.2) (layer "B.Cu") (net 19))
 (segment (start 150 145.5) (end 150 119.22) (width 0.2) (layer "B.Cu") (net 19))
 (segment (start 79.5 147.5) (end 79.5 148) (width 0.2) (layer "B.Cu") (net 19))
 (segment (start 102.42 69) (end 104.92 71.5) (width 0.2) (layer "F.Cu") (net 12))
 (segment (start 127 114) (end 101 88) (width 0.2) (layer "F.Cu") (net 12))
 (segment (start 101 88) (end 101 69) (width 0.2) (layer "F.Cu") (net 12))
 (segment (start 101 69) (end 102.42 69) (width 0.2) (layer "F.Cu") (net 12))
 (segment (start 147.32 114) (end 151 117.68) (width 0.2) (layer "B.Cu") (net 20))
 (segment (start 78.5 149.5) (end 69 140) (width 0.2) (layer "B.Cu") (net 20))
 (segment (start 69 140) (end 69 94.72) (width 0.2) (layer "B.Cu") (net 20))
 (segment (start 151 117.68) (end 151 149.5) (width 0.2) (layer "B.Cu") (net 20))
 (segment (start 69 94.72) (end 92.22 71.5) (width 0.2) (layer "B.Cu") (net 20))
 (segment (start 151 149.5) (end 78.5 149.5) (width 0.2) (layer "B.Cu") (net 20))
 (segment (start 255.5 103) (end 255.5 95.5) (width 0.2) (layer "F.Cu") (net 1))
 (via (at 255.5 95.5) (size 0.6) (drill 0.3) (layers "F.Cu" "B.Cu") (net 1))
 (segment (start 255.5 95.5) (end 255.5 31.04) (width 0.2) (layer "B.Cu") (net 1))
 (segment (start 255.5 31.04) (end 255.46 31) (width 0.2) (layer "B.Cu") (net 1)))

